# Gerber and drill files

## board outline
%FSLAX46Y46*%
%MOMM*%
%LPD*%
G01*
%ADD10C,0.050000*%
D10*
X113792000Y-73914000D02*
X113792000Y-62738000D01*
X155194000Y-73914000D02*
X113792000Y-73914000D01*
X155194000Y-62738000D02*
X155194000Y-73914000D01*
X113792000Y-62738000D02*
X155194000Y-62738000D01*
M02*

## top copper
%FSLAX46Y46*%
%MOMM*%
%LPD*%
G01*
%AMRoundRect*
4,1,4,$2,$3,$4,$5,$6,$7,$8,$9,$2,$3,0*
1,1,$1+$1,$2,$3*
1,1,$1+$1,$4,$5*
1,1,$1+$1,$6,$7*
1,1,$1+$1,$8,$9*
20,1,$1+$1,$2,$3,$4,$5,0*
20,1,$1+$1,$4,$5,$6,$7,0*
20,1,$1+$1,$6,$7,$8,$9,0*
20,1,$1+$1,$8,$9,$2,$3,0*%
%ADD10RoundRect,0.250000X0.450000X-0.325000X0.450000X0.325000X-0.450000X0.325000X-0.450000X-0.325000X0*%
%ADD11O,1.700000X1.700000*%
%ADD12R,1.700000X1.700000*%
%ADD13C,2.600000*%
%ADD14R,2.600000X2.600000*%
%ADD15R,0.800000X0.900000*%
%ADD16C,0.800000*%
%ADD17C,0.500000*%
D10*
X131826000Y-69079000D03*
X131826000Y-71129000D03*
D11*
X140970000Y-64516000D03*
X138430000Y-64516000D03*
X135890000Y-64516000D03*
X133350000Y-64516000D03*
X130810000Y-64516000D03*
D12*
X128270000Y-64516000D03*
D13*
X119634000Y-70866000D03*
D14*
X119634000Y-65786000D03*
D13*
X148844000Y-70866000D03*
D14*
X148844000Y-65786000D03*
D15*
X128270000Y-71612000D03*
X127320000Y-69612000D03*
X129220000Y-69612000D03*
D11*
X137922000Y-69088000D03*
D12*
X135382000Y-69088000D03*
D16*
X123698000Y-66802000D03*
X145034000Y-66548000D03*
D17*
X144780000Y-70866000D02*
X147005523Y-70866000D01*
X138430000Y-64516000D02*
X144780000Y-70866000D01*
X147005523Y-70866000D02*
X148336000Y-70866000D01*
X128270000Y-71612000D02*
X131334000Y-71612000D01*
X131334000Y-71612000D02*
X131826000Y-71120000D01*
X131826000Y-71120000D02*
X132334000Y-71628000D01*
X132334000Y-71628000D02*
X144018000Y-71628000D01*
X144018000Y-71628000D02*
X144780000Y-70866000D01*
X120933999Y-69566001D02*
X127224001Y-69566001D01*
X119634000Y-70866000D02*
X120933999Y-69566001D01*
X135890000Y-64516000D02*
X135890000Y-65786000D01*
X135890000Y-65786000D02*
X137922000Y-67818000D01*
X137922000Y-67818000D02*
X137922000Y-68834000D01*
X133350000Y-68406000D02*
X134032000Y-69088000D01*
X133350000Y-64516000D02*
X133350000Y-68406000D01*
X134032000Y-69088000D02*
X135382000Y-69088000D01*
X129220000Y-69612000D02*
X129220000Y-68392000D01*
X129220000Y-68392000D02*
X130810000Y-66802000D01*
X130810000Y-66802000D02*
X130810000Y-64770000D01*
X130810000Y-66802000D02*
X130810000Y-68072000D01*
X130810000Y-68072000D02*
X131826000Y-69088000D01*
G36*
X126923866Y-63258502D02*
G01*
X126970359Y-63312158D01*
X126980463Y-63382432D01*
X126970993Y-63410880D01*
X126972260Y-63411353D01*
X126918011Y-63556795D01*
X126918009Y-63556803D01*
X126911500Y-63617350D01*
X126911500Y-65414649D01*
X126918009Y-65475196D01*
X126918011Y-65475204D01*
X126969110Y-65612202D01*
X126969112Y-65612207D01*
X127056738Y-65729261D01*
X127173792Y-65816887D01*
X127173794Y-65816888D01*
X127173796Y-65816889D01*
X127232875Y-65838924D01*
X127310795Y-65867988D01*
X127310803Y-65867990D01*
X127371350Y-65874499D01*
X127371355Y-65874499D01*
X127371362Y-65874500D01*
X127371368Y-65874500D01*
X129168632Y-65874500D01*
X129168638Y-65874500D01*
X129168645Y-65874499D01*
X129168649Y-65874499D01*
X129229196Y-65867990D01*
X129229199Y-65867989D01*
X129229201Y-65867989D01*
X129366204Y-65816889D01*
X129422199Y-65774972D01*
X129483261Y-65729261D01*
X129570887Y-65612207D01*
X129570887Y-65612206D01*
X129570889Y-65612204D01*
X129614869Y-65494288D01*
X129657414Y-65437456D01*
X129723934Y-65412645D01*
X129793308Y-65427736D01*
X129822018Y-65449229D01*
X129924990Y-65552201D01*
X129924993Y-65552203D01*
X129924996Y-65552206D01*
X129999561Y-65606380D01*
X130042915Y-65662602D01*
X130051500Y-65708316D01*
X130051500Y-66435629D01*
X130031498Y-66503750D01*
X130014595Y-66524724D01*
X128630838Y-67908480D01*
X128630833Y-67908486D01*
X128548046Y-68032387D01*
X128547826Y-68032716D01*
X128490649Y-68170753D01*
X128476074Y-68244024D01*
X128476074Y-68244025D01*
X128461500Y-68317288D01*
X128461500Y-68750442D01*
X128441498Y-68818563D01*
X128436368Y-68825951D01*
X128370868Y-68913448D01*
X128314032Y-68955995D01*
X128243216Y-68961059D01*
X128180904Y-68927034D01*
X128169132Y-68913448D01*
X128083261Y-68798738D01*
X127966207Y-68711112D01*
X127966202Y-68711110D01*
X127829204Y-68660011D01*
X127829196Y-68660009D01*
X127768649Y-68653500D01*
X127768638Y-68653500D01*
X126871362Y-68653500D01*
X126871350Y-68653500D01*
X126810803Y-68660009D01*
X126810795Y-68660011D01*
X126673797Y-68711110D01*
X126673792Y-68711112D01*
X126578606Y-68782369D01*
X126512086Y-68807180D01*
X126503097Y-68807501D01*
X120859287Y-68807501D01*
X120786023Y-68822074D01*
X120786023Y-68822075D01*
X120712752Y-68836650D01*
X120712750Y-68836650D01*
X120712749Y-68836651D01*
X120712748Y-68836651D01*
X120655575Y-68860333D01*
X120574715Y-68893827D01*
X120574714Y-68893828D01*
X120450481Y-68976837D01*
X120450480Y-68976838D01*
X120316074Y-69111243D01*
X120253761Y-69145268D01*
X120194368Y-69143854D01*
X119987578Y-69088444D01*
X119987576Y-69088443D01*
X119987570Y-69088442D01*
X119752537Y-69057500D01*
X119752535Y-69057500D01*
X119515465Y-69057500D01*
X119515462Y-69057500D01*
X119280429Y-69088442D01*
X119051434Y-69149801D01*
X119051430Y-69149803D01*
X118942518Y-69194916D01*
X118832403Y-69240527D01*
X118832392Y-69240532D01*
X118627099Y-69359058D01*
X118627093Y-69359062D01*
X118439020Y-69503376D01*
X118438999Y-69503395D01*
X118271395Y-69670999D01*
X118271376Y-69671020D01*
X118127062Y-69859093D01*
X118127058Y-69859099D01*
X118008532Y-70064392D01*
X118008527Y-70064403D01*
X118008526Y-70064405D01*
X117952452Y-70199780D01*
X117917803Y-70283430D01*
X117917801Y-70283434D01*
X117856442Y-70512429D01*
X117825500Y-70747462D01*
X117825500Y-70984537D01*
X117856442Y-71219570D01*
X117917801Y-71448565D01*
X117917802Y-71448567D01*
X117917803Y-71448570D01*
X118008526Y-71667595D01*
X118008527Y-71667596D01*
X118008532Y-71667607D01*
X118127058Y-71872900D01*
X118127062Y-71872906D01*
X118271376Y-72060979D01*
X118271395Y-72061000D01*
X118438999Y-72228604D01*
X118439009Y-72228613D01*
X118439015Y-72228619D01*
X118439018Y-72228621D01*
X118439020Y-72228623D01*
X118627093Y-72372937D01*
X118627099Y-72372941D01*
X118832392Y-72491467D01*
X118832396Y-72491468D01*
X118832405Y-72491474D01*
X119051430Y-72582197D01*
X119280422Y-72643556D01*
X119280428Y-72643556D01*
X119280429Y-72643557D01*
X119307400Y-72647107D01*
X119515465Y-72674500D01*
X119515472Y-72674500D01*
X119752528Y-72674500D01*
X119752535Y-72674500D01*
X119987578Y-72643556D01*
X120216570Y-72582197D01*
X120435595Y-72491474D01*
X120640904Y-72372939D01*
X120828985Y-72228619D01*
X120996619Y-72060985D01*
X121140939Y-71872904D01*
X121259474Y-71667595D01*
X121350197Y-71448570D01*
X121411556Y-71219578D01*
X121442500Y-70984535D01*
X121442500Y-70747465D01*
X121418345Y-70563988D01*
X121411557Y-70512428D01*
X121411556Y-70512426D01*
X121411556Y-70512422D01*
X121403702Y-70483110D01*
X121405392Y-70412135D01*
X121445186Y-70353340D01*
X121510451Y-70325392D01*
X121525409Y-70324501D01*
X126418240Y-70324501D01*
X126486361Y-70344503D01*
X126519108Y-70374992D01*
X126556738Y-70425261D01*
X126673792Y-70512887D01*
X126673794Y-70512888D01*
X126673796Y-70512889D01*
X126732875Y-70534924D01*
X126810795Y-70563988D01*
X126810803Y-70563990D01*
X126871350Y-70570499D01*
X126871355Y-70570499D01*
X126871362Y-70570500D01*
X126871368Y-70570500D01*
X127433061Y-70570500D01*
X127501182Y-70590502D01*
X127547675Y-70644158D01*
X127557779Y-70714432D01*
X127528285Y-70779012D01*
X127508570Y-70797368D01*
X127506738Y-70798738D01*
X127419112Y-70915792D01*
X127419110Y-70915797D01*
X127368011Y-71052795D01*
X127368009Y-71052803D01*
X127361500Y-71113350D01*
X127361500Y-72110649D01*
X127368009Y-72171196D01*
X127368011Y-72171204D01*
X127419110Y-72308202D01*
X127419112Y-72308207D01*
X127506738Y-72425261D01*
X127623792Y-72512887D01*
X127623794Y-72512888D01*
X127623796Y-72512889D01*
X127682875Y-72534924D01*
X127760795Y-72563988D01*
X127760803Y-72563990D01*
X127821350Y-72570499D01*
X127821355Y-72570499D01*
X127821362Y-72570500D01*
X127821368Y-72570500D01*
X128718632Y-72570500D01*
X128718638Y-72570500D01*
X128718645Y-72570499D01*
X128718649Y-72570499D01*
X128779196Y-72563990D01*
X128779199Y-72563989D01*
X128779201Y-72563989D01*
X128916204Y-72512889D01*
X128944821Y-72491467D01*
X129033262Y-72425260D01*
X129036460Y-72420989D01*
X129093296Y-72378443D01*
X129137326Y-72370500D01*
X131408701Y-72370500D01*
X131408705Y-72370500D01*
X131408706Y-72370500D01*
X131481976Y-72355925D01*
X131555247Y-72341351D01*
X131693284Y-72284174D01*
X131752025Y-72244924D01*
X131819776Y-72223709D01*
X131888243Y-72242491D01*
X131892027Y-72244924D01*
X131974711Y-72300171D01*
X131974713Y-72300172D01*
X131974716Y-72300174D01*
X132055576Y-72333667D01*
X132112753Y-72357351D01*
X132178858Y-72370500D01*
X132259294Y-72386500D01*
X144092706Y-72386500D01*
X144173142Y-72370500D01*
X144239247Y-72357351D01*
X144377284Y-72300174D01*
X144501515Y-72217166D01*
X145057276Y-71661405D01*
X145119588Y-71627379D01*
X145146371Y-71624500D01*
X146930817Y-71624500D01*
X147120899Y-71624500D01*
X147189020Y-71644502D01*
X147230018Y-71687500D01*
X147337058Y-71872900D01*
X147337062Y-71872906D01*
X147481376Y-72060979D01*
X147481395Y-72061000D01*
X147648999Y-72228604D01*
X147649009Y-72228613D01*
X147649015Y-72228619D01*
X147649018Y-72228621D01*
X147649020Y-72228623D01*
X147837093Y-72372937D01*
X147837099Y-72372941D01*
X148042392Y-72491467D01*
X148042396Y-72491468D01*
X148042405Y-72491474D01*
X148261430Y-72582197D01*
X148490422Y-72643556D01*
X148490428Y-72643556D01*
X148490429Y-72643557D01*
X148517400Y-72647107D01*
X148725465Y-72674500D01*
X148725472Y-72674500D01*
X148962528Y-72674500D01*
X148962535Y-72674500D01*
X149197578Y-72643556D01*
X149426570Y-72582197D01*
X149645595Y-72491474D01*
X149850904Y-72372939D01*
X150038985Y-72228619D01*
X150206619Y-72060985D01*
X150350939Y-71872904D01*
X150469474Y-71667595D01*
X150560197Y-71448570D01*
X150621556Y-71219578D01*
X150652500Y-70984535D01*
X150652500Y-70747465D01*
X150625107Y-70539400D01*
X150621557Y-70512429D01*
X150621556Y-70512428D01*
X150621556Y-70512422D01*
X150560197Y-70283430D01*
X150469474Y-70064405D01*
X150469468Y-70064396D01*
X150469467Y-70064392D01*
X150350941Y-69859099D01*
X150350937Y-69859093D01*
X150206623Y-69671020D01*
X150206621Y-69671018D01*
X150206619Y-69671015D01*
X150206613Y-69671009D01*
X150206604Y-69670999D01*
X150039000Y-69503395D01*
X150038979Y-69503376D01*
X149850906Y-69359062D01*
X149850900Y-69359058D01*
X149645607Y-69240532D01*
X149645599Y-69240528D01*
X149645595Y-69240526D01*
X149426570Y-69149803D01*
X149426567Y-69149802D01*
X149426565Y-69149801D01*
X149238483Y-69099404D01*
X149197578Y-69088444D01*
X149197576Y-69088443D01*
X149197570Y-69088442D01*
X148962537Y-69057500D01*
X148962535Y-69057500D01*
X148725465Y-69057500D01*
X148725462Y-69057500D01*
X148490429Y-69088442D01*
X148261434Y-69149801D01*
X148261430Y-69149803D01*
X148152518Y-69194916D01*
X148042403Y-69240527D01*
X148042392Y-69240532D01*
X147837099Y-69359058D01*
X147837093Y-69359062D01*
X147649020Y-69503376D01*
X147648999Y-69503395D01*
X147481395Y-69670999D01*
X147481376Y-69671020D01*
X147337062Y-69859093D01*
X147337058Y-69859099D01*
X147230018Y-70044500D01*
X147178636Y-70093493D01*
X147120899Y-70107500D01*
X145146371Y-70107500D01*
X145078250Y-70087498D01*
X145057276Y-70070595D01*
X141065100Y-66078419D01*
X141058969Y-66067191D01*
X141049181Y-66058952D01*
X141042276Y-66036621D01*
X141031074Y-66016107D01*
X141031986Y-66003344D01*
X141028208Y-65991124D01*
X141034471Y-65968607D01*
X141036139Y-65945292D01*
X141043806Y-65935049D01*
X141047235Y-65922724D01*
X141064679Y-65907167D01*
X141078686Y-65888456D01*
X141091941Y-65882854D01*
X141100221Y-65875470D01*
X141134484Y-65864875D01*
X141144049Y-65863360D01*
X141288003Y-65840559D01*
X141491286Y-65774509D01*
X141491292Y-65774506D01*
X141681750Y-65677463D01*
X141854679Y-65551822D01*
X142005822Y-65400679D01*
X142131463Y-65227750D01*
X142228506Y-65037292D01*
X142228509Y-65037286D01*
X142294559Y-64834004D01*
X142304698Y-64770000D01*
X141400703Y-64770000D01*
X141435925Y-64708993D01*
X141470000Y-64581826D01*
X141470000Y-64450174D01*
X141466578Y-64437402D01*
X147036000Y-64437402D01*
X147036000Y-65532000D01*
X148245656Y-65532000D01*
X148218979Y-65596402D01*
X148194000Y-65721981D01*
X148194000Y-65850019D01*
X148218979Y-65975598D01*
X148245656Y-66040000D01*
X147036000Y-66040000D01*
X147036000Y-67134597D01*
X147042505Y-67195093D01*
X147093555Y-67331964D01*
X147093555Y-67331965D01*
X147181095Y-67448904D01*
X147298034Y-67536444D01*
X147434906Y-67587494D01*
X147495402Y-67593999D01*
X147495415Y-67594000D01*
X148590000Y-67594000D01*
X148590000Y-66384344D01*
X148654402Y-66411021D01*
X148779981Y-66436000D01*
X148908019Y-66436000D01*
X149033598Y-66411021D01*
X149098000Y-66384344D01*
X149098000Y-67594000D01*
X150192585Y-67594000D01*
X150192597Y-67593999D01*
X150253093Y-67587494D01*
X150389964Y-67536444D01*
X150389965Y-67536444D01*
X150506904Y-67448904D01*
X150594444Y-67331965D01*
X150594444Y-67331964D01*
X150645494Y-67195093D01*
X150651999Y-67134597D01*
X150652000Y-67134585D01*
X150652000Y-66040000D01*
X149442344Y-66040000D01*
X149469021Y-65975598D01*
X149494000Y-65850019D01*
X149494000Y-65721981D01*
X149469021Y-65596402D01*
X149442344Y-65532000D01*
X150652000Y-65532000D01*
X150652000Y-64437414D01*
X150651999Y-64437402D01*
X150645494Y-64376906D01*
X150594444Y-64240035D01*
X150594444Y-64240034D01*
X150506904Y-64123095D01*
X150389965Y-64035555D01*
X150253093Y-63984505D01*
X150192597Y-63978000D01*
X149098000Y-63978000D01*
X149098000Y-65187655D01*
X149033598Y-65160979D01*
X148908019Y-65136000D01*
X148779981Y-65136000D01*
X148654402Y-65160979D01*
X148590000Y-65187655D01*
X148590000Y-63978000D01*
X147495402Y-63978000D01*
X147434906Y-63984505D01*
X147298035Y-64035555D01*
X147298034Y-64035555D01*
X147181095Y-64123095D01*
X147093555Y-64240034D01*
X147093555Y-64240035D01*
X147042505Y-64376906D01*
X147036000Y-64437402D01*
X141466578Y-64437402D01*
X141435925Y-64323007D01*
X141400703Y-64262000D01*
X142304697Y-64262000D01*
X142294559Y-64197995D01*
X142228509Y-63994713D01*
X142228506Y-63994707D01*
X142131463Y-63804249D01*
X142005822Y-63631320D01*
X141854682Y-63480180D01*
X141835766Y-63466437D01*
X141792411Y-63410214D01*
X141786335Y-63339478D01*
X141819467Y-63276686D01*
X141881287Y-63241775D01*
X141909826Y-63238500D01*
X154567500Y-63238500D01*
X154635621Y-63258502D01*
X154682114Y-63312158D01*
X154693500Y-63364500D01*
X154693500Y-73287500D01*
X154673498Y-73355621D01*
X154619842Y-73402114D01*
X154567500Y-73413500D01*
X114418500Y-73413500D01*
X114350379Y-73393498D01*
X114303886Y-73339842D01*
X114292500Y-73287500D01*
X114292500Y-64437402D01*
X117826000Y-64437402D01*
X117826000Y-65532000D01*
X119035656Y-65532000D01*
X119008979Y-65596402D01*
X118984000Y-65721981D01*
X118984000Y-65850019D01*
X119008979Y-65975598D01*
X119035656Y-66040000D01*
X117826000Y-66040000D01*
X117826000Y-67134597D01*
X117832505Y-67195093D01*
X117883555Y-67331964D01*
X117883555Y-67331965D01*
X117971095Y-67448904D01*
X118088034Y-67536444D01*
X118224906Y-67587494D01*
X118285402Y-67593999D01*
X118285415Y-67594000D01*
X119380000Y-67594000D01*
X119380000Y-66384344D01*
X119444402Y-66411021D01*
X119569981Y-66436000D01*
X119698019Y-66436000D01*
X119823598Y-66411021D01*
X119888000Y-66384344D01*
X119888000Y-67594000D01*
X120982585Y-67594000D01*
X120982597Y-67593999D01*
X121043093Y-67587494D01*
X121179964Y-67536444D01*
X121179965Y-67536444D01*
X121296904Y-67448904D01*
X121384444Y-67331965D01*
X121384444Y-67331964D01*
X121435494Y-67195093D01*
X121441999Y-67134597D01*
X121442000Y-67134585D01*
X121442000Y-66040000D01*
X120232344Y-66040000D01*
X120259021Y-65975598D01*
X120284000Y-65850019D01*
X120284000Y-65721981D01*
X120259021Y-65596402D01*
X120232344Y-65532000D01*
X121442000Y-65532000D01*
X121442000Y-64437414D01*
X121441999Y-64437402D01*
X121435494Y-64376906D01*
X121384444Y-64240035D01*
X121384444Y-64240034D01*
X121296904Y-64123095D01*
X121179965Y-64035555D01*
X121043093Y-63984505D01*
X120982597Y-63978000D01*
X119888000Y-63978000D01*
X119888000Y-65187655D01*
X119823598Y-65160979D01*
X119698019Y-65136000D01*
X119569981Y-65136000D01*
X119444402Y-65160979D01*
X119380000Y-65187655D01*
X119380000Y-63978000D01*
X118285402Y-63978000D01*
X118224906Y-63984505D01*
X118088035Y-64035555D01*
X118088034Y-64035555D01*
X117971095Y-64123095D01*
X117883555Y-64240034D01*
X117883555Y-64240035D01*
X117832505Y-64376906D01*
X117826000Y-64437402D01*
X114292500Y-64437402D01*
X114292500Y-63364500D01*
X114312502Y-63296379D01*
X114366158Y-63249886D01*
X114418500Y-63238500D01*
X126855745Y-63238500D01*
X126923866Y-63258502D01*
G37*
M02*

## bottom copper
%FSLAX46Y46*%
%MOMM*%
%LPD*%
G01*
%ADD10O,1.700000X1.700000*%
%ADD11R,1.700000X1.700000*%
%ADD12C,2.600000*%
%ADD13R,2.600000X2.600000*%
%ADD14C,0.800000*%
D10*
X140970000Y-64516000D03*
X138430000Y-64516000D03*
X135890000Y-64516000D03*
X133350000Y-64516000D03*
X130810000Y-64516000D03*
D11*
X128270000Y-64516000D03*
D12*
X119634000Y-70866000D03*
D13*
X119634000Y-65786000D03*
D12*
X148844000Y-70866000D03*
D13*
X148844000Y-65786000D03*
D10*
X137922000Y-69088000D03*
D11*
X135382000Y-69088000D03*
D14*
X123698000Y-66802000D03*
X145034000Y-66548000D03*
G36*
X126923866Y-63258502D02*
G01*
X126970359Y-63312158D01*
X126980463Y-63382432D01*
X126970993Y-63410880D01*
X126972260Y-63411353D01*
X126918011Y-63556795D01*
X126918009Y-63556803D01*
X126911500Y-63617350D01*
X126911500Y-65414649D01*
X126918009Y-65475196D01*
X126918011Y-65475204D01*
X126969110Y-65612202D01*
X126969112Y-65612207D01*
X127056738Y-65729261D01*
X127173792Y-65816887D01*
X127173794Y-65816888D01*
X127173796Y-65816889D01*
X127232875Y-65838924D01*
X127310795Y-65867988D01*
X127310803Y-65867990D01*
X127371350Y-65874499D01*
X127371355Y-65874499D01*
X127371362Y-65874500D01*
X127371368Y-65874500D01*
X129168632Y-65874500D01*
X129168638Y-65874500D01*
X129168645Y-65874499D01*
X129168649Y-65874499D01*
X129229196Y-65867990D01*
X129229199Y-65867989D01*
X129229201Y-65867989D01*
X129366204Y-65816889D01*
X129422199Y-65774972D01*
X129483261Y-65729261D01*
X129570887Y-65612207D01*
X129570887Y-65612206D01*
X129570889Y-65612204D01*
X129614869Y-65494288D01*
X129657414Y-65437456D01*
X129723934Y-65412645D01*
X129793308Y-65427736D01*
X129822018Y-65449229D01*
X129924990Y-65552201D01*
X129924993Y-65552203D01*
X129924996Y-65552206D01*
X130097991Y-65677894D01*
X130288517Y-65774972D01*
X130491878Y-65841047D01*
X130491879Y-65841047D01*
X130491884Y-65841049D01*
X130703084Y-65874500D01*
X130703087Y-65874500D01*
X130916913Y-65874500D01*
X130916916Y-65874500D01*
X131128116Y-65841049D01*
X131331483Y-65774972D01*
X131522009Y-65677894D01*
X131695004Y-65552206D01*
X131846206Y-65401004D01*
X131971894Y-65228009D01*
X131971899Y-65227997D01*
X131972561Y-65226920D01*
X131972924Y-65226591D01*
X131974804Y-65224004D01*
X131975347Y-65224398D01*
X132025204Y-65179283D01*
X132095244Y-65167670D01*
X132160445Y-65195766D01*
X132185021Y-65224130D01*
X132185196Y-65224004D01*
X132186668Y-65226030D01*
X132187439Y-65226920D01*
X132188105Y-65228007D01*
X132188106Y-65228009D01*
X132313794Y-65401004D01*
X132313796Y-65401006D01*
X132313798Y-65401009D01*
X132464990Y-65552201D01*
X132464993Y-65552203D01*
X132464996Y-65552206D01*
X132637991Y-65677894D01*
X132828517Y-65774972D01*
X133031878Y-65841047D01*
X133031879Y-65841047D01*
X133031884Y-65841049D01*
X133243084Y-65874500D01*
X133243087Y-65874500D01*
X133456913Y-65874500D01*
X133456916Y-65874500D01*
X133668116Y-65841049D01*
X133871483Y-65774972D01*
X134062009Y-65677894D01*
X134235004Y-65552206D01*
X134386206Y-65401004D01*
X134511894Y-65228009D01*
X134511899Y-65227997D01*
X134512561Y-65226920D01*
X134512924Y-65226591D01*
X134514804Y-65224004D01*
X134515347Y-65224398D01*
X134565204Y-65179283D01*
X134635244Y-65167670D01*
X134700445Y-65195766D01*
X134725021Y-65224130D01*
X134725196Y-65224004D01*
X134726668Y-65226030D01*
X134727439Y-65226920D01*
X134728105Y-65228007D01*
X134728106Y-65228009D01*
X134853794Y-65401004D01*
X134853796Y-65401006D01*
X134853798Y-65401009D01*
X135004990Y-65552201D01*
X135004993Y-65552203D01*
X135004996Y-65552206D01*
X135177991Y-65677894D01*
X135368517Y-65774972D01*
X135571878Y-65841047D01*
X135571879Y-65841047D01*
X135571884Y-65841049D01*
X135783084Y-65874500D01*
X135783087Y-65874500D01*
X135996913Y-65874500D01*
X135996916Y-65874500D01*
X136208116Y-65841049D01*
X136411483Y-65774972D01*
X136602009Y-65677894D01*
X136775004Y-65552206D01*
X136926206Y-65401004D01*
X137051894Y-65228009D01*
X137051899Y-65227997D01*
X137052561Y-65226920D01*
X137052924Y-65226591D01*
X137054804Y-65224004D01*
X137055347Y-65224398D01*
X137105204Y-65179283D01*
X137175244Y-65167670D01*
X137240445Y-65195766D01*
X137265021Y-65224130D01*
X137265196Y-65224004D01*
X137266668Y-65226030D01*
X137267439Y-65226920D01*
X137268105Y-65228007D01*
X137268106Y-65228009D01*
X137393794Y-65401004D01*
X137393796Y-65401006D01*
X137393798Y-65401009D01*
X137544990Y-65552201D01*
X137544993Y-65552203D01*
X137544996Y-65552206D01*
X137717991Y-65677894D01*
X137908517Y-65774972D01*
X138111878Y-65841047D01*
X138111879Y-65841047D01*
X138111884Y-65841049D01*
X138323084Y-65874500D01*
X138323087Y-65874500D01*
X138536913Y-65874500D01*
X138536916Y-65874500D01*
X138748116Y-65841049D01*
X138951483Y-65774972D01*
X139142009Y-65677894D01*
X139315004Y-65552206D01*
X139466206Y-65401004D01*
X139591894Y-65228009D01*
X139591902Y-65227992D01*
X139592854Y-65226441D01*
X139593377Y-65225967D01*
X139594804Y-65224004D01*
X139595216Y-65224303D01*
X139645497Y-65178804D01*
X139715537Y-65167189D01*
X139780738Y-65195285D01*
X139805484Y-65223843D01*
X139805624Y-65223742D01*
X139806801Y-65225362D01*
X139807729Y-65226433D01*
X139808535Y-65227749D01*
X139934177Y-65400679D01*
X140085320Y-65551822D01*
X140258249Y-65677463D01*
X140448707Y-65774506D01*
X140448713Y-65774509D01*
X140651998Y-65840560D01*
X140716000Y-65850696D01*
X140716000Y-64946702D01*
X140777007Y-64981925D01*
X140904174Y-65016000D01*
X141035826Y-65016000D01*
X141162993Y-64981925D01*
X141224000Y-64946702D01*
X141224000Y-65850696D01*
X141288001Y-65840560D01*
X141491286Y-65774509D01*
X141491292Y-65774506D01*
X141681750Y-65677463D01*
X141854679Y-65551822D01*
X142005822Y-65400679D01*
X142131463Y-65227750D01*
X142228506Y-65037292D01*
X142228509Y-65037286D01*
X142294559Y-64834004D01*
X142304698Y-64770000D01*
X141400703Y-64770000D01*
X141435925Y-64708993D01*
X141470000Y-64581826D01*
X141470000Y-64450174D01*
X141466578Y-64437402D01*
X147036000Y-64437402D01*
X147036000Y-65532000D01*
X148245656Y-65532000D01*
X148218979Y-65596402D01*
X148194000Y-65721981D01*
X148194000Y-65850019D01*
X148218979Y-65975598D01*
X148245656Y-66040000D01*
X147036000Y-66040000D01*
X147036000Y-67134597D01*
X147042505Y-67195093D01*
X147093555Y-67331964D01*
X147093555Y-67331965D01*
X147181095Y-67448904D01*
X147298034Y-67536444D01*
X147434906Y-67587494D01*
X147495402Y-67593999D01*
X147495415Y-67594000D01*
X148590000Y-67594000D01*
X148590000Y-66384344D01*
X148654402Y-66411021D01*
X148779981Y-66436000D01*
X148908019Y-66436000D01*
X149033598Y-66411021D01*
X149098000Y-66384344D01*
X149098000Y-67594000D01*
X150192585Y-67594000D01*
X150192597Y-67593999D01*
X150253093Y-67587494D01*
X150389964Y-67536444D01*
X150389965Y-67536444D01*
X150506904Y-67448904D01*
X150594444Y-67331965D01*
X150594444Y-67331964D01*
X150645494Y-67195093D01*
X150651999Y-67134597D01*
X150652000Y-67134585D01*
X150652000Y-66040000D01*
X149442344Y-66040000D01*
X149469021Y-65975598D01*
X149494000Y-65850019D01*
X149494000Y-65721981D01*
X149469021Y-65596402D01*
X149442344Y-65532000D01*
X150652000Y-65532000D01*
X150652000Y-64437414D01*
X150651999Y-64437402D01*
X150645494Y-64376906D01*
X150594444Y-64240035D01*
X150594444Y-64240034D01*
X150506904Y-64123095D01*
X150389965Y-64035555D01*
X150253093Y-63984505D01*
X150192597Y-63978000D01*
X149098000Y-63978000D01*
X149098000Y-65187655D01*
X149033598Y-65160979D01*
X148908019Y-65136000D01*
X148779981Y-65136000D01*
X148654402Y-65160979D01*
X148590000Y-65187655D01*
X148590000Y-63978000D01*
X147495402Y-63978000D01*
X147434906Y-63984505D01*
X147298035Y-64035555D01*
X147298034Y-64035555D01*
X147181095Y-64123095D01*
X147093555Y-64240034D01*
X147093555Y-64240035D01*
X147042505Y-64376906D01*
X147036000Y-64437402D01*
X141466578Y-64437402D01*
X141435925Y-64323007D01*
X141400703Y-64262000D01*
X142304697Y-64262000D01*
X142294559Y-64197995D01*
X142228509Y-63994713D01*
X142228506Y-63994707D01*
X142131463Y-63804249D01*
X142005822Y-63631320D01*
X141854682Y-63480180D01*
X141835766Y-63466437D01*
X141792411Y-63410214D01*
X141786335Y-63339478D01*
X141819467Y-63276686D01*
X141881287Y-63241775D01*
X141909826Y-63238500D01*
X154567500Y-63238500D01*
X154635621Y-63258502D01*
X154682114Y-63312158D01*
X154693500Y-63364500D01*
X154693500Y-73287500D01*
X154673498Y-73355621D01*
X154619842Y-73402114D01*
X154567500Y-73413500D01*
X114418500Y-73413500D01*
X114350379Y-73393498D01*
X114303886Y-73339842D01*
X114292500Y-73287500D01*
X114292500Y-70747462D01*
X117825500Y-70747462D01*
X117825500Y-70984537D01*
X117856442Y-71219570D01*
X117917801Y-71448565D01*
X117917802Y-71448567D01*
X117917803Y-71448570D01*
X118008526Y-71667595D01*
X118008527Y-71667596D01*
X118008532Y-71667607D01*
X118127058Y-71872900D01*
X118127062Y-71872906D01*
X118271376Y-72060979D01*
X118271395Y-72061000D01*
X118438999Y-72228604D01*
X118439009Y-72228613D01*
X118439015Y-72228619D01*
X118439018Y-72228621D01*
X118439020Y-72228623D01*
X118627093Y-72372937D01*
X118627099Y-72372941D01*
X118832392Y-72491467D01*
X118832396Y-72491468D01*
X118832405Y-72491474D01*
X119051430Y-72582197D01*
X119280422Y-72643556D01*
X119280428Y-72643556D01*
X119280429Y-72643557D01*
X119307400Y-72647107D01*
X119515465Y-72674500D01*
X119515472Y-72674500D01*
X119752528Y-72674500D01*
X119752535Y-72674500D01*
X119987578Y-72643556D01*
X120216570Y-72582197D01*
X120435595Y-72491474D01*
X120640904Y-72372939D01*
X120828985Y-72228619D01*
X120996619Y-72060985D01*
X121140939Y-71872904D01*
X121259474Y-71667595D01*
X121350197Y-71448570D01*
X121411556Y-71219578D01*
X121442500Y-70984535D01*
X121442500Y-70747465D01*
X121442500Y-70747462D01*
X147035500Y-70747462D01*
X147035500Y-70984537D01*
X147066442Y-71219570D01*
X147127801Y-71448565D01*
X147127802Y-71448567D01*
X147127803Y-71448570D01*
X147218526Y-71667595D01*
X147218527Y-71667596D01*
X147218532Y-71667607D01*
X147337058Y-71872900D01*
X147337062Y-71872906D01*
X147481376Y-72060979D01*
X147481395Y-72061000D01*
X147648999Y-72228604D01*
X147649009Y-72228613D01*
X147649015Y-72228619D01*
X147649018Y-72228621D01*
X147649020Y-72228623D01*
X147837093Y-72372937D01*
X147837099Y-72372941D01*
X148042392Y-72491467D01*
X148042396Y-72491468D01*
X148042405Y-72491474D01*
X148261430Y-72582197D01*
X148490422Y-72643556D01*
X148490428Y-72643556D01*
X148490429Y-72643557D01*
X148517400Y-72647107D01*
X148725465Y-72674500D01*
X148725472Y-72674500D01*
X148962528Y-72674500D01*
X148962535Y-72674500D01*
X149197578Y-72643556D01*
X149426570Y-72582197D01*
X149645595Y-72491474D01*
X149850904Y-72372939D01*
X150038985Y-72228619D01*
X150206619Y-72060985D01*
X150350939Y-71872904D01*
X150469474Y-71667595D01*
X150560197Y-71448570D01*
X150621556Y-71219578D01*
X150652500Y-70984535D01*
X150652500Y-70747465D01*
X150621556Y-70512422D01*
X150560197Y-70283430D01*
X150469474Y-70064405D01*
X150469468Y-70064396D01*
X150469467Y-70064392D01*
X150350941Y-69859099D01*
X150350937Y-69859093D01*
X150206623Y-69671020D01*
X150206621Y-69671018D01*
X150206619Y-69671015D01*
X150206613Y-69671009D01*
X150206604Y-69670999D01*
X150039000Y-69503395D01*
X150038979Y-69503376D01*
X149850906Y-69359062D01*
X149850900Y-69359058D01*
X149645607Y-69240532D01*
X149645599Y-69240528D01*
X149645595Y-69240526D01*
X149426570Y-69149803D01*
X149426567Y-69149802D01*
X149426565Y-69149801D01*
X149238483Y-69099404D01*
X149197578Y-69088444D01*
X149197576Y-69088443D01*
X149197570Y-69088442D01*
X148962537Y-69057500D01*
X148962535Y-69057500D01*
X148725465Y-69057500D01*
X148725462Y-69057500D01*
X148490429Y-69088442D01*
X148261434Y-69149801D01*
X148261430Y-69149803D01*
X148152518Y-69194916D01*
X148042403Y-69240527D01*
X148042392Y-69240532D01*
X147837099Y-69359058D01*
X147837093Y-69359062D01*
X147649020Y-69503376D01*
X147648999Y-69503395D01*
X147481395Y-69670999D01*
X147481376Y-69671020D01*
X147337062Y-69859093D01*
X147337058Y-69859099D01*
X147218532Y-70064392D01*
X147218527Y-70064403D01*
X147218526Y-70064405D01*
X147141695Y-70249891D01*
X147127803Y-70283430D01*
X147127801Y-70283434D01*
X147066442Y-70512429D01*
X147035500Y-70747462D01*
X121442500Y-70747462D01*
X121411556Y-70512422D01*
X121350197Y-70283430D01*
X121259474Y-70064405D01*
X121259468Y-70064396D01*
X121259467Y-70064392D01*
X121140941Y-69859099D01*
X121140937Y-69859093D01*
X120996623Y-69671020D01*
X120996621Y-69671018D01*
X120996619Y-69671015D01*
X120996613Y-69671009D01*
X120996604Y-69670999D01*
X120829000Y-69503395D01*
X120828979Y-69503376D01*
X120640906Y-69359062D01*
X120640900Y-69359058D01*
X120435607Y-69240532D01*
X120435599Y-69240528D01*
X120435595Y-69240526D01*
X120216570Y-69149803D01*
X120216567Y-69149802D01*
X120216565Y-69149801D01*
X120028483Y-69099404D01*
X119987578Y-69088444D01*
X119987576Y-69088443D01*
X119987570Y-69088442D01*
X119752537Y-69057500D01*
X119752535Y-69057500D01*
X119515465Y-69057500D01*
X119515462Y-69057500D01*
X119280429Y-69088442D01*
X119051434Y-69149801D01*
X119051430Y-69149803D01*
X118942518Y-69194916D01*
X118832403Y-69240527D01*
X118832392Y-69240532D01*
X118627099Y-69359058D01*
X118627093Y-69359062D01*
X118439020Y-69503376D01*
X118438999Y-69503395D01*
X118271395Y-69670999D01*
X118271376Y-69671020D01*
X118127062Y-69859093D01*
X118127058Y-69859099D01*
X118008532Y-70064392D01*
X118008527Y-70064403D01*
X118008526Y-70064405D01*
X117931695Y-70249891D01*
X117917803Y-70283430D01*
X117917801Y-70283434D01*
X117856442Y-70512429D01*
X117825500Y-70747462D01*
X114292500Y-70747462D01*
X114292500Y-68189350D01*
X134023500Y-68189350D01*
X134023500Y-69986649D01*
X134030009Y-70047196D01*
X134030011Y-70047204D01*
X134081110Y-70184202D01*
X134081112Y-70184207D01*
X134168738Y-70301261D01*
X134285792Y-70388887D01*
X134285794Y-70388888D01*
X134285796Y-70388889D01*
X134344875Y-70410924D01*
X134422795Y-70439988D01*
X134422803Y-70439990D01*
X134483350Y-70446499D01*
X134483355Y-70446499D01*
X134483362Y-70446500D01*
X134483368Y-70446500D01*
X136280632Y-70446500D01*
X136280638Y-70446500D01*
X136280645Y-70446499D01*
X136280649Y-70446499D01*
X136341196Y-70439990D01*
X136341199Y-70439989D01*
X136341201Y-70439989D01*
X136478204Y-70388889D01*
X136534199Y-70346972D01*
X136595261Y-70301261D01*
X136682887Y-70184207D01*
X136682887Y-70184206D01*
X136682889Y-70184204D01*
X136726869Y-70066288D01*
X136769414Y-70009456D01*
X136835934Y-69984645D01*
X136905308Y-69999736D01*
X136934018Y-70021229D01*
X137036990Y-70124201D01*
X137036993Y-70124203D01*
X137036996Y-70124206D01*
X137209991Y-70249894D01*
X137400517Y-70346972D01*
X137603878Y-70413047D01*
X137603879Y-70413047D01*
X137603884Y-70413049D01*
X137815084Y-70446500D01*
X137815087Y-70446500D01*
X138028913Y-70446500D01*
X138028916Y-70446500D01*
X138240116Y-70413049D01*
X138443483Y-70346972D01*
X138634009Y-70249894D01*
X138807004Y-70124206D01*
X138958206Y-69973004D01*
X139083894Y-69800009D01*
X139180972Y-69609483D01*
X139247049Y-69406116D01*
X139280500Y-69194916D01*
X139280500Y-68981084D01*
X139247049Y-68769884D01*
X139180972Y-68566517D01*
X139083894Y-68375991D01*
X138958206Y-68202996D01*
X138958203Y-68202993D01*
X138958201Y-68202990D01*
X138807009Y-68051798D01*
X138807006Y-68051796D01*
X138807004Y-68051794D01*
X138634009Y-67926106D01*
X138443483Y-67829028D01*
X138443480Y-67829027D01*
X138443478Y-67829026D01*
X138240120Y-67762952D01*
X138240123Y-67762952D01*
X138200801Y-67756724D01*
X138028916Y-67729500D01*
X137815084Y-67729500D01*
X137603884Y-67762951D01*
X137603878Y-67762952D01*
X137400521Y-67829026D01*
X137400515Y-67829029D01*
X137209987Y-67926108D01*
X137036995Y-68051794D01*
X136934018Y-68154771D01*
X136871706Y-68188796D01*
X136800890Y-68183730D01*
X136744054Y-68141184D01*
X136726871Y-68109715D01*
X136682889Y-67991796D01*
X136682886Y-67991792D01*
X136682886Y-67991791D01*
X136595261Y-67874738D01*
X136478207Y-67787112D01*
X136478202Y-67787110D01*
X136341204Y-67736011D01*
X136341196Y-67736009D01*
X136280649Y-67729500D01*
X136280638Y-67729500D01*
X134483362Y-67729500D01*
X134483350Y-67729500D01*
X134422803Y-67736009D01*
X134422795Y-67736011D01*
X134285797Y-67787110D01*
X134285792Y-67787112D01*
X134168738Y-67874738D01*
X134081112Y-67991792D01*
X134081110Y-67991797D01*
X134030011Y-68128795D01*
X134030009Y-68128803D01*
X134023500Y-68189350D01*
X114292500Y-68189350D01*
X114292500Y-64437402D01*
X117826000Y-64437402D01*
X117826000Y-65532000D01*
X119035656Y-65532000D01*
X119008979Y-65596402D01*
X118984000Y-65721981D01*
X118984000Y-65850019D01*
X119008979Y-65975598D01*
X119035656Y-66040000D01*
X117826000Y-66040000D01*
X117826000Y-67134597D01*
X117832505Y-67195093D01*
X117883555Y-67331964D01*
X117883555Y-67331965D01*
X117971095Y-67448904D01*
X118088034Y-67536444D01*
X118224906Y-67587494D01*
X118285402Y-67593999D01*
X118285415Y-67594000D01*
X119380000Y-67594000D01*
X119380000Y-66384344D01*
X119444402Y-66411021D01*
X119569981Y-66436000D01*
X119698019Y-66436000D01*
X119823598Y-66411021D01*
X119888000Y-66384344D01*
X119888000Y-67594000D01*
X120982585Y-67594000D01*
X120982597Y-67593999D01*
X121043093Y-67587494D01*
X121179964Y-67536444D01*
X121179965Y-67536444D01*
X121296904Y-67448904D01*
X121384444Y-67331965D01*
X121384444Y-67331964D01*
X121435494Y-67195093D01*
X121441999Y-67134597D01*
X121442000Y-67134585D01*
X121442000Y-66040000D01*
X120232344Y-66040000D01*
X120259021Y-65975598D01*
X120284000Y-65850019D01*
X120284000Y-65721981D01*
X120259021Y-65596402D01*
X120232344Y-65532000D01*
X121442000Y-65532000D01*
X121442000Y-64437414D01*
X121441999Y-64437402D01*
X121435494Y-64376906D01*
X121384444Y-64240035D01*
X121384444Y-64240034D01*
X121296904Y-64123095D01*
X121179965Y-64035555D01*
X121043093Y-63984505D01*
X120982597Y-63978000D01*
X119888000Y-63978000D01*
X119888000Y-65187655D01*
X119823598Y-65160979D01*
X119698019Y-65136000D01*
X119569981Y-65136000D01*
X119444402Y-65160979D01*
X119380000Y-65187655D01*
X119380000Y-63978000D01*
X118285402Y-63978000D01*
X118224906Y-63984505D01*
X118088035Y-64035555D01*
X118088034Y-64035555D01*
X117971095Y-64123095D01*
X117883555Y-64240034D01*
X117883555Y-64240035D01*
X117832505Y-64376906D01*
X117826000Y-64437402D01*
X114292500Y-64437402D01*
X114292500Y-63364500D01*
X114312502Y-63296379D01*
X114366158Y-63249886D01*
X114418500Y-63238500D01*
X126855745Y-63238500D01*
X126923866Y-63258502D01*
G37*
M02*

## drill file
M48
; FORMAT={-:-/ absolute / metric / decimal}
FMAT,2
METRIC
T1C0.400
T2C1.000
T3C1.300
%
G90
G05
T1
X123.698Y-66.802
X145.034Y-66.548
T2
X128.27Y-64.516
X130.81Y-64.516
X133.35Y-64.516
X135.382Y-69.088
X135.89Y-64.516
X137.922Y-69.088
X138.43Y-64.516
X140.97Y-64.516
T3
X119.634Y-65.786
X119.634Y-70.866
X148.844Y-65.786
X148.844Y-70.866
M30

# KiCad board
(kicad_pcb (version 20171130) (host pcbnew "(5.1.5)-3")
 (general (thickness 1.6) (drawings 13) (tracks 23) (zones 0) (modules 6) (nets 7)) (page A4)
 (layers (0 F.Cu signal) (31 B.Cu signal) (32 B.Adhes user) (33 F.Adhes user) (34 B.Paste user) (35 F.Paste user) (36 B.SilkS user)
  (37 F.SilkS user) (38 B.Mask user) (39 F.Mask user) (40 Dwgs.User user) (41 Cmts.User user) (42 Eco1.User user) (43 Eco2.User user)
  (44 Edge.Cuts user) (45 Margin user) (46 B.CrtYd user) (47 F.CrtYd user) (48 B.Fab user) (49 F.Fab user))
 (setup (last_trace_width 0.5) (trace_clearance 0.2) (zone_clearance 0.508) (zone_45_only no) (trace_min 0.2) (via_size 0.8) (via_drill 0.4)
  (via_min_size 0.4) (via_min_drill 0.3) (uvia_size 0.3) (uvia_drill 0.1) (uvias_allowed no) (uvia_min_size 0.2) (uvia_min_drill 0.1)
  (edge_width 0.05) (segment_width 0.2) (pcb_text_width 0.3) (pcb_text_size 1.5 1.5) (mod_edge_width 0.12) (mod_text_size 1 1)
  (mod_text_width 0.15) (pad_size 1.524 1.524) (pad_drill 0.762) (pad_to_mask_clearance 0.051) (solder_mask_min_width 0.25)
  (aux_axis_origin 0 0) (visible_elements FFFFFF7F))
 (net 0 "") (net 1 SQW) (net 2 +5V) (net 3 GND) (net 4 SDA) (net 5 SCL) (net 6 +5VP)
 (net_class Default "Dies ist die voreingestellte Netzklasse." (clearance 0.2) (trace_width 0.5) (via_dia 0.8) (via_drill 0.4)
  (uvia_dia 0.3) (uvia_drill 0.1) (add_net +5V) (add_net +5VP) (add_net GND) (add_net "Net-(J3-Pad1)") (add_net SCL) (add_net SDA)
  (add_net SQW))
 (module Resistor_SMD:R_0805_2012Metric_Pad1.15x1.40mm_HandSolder (layer F.Cu) (at 131.826 70.104 90)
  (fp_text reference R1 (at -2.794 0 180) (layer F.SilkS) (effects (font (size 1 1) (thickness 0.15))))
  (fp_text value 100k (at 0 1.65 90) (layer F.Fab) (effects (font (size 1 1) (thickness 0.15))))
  (pad 2 smd roundrect (at 1.025 0 90) (size 1.15 1.4) (layers F.Cu F.Paste F.Mask) (roundrect_rratio 0.217391) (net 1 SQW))
  (pad 1 smd roundrect (at -1.025 0 90) (size 1.15 1.4) (layers F.Cu F.Paste F.Mask) (roundrect_rratio 0.217391) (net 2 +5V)))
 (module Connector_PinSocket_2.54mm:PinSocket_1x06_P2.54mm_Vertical (layer F.Cu) (at 128.27 64.516 90)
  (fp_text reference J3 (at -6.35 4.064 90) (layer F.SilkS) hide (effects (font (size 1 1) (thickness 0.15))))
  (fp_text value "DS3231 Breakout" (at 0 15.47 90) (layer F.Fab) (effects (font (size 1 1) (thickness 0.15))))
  (pad 6 thru_hole oval (at 0 12.7 90) (size 1.7 1.7) (drill 1) (layers *.Cu *.Mask) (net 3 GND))
  (pad 5 thru_hole oval (at 0 10.16 90) (size 1.7 1.7) (drill 1) (layers *.Cu *.Mask) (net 2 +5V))
  (pad 4 thru_hole oval (at 0 7.62 90) (size 1.7 1.7) (drill 1) (layers *.Cu *.Mask) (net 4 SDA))
  (pad 3 thru_hole oval (at 0 5.08 90) (size 1.7 1.7) (drill 1) (layers *.Cu *.Mask) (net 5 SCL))
  (pad 2 thru_hole oval (at 0 2.54 90) (size 1.7 1.7) (drill 1) (layers *.Cu *.Mask) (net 1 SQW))
  (pad 1 thru_hole rect (at 0 0 90) (size 1.7 1.7) (drill 1) (layers *.Cu *.Mask)))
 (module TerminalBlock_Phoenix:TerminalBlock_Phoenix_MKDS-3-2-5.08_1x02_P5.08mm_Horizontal (layer F.Cu) (at 119.634 65.786 270)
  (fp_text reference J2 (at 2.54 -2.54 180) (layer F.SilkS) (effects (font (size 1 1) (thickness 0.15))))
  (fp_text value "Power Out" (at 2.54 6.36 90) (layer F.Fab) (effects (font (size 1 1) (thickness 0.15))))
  (pad 2 thru_hole circle (at 5.08 0 270) (size 2.6 2.6) (drill 1.3) (layers *.Cu *.Mask) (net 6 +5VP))
  (pad 1 thru_hole rect (at 0 0 270) (size 2.6 2.6) (drill 1.3) (layers *.Cu *.Mask) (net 3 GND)))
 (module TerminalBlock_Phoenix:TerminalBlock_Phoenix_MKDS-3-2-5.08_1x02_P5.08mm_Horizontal (layer F.Cu) (at 148.844 65.786 270)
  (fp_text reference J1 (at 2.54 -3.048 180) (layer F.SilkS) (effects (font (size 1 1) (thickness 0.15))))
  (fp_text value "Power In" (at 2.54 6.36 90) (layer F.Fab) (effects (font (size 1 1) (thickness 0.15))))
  (pad 2 thru_hole circle (at 5.08 0 270) (size 2.6 2.6) (drill 1.3) (layers *.Cu *.Mask) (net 2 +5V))
  (pad 1 thru_hole rect (at 0 0 270) (size 2.6 2.6) (drill 1.3) (layers *.Cu *.Mask) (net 3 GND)))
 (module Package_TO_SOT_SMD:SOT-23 (layer F.Cu) (at 128.27 70.612 270)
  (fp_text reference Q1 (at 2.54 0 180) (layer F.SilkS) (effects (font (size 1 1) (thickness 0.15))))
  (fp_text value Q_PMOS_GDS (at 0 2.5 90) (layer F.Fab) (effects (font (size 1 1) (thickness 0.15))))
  (pad 3 smd rect (at 1 0 270) (size 0.9 0.8) (layers F.Cu F.Paste F.Mask) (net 2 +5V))
  (pad 2 smd rect (at -1 0.95 270) (size 0.9 0.8) (layers F.Cu F.Paste F.Mask) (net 6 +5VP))
  (pad 1 smd rect (at -1 -0.95 270) (size 0.9 0.8) (layers F.Cu F.Paste F.Mask) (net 1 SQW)))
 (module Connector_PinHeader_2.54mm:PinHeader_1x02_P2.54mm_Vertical (layer F.Cu) (at 135.382 69.088 90)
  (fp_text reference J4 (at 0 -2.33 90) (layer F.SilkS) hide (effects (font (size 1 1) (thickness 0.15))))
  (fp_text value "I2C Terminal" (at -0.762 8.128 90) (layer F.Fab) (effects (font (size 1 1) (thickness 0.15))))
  (pad 2 thru_hole oval (at 0 2.54 90) (size 1.7 1.7) (drill 1) (layers *.Cu *.Mask) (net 4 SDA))
  (pad 1 thru_hole rect (at 0 0 90) (size 1.7 1.7) (drill 1) (layers *.Cu *.Mask) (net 5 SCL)))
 (gr_line (start 113.792 73.914) (end 113.792 62.738) (layer Edge.Cuts) (width 0.05))
 (gr_line (start 155.194 73.914) (end 113.792 73.914) (layer Edge.Cuts) (width 0.05))
 (gr_line (start 155.194 62.738) (end 155.194 73.914) (layer Edge.Cuts) (width 0.05))
 (gr_line (start 113.792 62.738) (end 155.194 62.738) (layer Edge.Cuts) (width 0.05))
 (via (at 123.698 66.802) (size 0.8) (drill 0.4) (layers F.Cu B.Cu) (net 3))
 (via (at 145.034 66.548) (size 0.8) (drill 0.4) (layers F.Cu B.Cu) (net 3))
 (segment (start 144.78 70.866) (end 147.005523 70.866) (width 0.5) (layer F.Cu) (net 2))
 (segment (start 138.43 64.516) (end 144.78 70.866) (width 0.5) (layer F.Cu) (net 2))
 (segment (start 147.005523 70.866) (end 148.336 70.866) (width 0.5) (layer F.Cu) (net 2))
 (segment (start 128.27 71.612) (end 131.334 71.612) (width 0.5) (layer F.Cu) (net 2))
 (segment (start 131.334 71.612) (end 131.826 71.12) (width 0.5) (layer F.Cu) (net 2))
 (segment (start 131.826 71.12) (end 132.334 71.628) (width 0.5) (layer F.Cu) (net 2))
 (segment (start 132.334 71.628) (end 144.018 71.628) (width 0.5) (layer F.Cu) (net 2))
 (segment (start 144.018 71.628) (end 144.78 70.866) (width 0.5) (layer F.Cu) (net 2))
 (segment (start 120.933999 69.566001) (end 127.224001 69.566001) (width 0.5) (layer F.Cu) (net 6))
 (segment (start 119.634 70.866) (end 120.933999 69.566001) (width 0.5) (layer F.Cu) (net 6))
 (segment (start 135.89 64.516) (end 135.89 65.786) (width 0.5) (layer F.Cu) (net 4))
 (segment (start 135.89 65.786) (end 137.922 67.818) (width 0.5) (layer F.Cu) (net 4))
 (segment (start 137.922 67.818) (end 137.922 68.834) (width 0.5) (layer F.Cu) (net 4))
 (segment (start 133.35 68.406) (end 134.032 69.088) (width 0.5) (layer F.Cu) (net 5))
 (segment (start 133.35 64.516) (end 133.35 68.406) (width 0.5) (layer F.Cu) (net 5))
 (segment (start 134.032 69.088) (end 135.382 69.088) (width 0.5) (layer F.Cu) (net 5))
 (segment (start 129.22 69.612) (end 129.22 68.392) (width 0.5) (layer F.Cu) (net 1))
 (segment (start 129.22 68.392) (end 130.81 66.802) (width 0.5) (layer F.Cu) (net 1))
 (segment (start 130.81 66.802) (end 130.81 64.77) (width 0.5) (layer F.Cu) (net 1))
 (segment (start 130.81 66.802) (end 130.81 68.072) (width 0.5) (layer F.Cu) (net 1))
 (segment (start 130.81 68.072) (end 131.826 69.088) (width 0.5) (layer F.Cu) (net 1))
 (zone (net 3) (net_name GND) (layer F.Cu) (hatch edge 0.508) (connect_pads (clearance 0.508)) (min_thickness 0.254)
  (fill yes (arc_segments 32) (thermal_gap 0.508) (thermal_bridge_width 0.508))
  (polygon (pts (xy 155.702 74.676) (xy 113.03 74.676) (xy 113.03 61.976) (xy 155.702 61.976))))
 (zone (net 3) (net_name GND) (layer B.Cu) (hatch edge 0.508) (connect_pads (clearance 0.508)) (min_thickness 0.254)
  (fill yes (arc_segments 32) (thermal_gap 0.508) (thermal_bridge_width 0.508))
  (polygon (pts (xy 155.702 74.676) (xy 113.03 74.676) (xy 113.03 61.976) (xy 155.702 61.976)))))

